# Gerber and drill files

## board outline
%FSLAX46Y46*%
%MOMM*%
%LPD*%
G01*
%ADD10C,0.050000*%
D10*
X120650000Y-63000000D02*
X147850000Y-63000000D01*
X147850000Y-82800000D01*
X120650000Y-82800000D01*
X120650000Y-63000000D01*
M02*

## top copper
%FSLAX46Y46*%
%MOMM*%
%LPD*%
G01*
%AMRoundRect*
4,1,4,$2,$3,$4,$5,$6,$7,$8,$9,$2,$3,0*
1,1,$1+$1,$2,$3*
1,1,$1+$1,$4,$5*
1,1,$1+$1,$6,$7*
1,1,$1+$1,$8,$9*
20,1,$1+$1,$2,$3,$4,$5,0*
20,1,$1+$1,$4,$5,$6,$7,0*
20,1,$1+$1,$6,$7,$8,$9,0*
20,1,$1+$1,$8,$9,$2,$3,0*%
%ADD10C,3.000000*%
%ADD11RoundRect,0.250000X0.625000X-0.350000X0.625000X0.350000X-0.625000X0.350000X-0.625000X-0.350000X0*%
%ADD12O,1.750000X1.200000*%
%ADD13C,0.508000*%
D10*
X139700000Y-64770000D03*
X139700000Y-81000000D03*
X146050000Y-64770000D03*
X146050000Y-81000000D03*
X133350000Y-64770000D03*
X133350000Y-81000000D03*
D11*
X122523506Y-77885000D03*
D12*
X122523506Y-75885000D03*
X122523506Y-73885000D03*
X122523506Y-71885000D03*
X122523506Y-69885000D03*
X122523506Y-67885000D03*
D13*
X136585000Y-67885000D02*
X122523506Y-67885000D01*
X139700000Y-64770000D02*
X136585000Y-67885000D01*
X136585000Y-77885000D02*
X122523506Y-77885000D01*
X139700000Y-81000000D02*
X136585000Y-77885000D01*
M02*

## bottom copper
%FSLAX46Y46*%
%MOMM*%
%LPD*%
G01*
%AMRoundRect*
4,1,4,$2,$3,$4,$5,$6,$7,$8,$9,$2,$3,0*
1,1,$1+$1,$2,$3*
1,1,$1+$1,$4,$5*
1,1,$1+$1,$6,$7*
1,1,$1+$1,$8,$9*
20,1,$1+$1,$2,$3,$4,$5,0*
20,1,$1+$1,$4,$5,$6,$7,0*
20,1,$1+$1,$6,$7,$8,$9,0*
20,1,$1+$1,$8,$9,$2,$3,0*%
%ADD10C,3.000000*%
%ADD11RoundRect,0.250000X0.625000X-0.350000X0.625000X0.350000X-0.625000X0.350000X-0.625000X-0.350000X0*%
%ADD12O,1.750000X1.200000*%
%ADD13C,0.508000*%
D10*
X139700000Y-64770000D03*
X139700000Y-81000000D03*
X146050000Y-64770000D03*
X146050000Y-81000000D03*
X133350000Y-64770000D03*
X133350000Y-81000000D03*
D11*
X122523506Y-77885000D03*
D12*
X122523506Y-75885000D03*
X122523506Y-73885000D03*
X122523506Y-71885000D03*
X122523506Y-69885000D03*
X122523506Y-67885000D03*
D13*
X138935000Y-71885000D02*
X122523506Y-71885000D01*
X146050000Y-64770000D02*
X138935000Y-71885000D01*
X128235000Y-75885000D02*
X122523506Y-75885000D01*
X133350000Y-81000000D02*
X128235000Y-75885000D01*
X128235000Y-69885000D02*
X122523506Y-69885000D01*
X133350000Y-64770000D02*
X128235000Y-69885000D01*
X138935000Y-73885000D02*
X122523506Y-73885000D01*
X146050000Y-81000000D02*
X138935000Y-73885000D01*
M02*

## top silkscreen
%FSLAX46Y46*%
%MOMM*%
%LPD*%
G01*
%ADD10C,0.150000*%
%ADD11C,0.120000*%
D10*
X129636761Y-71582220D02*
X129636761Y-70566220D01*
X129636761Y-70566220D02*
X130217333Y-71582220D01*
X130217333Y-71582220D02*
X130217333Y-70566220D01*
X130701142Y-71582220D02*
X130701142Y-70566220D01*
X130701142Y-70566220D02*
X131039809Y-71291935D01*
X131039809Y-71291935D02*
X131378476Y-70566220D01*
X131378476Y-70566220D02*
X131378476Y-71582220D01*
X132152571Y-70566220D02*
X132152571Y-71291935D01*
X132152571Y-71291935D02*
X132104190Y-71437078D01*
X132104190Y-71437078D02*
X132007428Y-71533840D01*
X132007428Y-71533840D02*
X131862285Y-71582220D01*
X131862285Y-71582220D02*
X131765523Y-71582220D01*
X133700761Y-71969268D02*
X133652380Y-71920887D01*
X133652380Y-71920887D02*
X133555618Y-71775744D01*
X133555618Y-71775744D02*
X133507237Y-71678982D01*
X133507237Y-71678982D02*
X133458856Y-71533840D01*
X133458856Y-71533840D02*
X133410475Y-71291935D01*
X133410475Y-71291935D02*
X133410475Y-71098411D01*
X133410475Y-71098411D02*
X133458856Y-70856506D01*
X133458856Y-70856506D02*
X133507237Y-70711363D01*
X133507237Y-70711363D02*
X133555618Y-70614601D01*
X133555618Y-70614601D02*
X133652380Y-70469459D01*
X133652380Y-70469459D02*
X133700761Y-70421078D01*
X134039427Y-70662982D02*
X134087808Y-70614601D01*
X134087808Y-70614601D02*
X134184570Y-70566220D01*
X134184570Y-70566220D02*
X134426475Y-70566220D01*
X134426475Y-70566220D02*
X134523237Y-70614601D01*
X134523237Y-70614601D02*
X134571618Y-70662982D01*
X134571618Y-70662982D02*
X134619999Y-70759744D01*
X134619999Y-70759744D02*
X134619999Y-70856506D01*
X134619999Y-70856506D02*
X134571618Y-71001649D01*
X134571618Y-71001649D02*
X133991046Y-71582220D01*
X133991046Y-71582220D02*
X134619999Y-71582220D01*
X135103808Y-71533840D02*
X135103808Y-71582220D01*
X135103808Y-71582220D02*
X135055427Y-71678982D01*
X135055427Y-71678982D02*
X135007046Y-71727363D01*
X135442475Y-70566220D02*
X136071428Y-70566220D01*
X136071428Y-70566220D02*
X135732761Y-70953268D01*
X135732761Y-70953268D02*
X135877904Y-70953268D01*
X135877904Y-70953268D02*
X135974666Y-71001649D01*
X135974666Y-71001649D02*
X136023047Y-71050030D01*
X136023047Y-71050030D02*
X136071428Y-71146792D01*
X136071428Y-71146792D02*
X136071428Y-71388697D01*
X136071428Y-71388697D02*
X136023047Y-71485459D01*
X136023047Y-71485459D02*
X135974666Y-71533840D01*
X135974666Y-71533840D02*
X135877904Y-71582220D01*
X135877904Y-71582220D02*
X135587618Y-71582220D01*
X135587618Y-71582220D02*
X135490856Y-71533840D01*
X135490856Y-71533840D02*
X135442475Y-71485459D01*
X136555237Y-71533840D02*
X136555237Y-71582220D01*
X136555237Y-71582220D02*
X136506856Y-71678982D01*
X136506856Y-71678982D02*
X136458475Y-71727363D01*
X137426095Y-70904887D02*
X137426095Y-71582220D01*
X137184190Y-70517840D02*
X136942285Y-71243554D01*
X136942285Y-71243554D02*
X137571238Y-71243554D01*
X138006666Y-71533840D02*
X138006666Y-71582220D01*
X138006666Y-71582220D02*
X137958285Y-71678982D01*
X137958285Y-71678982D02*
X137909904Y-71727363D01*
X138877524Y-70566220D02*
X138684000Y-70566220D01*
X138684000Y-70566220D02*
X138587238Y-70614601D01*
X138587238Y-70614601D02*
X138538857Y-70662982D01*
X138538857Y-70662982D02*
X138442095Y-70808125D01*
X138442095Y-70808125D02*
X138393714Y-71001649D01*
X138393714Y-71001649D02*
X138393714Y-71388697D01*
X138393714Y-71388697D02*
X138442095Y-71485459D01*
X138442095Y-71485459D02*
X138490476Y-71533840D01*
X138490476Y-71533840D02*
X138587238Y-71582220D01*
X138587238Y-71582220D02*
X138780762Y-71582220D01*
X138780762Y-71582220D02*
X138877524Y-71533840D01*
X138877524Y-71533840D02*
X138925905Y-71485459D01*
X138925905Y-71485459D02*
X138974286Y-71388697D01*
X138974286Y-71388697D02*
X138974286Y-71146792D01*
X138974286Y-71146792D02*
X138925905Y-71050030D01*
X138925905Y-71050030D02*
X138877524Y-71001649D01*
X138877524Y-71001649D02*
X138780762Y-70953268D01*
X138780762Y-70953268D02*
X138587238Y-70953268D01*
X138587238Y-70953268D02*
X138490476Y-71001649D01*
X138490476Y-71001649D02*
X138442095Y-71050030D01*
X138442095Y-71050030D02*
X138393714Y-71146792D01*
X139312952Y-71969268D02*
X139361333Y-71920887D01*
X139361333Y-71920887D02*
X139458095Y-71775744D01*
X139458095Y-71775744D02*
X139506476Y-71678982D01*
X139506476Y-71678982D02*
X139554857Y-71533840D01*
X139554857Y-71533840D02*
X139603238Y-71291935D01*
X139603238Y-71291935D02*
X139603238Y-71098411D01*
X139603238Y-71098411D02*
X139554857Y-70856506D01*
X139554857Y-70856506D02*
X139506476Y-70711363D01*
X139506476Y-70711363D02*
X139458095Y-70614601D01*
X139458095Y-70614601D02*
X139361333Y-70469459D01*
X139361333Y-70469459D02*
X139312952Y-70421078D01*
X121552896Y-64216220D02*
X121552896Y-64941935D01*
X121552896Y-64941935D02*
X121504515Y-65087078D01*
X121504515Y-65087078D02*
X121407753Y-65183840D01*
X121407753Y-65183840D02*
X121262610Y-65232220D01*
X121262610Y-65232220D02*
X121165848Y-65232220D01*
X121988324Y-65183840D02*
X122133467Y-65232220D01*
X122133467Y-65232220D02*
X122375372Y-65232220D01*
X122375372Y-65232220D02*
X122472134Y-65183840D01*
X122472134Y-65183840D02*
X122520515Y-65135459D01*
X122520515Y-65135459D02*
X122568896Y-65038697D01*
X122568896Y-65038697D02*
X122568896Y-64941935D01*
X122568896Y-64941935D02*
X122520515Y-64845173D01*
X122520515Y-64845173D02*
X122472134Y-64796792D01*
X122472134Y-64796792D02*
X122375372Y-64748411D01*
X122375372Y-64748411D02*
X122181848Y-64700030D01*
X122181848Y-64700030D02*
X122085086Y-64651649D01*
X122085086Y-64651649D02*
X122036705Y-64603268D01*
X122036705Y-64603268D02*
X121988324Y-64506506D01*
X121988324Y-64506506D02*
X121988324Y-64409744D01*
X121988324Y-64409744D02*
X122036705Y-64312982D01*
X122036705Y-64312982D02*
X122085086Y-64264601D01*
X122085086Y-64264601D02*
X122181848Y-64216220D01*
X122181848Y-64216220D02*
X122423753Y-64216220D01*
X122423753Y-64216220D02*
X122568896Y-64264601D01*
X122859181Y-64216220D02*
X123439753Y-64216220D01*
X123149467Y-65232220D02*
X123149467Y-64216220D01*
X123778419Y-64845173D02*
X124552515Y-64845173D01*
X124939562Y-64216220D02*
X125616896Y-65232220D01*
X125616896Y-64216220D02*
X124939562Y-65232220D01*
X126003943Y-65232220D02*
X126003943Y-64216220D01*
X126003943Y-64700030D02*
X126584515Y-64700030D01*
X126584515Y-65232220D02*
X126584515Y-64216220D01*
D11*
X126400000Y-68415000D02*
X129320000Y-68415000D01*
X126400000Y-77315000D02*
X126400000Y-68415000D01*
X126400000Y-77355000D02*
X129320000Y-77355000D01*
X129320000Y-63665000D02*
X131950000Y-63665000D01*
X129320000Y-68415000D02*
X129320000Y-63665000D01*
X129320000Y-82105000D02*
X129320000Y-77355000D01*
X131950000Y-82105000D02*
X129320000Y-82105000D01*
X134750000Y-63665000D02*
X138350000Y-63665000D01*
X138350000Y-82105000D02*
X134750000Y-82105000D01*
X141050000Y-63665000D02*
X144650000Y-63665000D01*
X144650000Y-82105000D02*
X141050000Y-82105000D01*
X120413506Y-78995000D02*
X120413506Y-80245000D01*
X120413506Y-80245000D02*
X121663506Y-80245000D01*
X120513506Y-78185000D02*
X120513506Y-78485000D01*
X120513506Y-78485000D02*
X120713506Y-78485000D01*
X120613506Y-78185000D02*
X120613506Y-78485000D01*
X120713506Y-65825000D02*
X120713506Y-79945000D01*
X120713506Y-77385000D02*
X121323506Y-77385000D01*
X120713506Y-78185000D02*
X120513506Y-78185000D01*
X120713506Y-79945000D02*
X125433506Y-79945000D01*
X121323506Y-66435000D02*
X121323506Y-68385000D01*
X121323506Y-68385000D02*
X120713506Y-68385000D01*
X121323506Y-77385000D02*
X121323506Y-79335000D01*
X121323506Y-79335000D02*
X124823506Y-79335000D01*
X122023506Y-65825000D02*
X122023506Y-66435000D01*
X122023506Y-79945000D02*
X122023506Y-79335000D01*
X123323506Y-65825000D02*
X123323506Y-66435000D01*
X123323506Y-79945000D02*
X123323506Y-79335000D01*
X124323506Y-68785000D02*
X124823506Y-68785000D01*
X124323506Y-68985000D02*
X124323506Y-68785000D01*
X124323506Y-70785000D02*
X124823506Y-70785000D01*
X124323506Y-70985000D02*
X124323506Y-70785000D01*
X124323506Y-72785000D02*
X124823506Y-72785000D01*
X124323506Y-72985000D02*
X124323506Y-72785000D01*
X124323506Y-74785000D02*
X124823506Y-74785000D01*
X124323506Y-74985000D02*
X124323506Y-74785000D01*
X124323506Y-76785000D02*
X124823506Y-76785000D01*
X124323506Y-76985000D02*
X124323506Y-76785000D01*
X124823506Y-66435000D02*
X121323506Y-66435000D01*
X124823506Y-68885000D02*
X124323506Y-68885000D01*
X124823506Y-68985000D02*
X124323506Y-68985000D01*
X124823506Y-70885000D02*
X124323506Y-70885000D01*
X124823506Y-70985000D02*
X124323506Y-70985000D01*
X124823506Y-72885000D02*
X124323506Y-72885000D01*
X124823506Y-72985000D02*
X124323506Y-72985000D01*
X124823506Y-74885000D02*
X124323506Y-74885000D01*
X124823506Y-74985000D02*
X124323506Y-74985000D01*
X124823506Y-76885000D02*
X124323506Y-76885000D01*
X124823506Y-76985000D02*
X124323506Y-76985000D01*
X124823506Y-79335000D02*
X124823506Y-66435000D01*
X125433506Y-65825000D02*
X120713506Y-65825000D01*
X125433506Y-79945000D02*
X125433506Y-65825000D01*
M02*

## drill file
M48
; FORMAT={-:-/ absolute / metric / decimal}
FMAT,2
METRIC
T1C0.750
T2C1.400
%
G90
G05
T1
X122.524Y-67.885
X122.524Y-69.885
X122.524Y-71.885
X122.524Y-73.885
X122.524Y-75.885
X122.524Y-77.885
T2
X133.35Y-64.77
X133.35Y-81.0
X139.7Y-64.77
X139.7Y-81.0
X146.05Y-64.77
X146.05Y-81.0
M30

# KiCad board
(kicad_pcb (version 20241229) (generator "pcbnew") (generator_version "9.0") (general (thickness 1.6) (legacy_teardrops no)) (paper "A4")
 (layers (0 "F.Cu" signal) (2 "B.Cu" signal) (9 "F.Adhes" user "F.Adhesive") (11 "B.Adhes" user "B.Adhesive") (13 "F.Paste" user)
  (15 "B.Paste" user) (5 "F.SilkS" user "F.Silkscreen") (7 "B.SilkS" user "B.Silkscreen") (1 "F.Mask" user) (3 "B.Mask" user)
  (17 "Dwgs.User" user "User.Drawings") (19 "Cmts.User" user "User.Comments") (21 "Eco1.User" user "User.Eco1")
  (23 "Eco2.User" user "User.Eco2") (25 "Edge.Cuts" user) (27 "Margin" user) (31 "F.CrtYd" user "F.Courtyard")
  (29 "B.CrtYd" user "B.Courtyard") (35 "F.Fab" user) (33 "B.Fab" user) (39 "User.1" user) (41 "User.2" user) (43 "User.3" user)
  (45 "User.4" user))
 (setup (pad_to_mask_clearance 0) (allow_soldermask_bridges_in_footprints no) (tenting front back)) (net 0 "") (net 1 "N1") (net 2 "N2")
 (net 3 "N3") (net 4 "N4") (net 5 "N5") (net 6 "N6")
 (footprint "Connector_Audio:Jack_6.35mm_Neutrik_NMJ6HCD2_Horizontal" (layer "F.Cu") (at 133.35 64.77)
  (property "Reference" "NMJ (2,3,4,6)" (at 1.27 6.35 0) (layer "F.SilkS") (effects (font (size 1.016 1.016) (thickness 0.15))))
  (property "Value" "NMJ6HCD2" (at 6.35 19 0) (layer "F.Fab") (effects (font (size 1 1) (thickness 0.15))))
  (fp_line (start -6.95 3.645) (end -4.03 3.645) (stroke (width 0.12) (type solid)) (layer "F.SilkS"))
  (fp_line (start -6.95 12.545) (end -6.95 3.645) (stroke (width 0.12) (type solid)) (layer "F.SilkS"))
  (fp_line (start -6.95 12.585) (end -4.03 12.585) (stroke (width 0.12) (type solid)) (layer "F.SilkS"))
  (fp_line (start -4.03 -1.105) (end -1.4 -1.105) (stroke (width 0.12) (type solid)) (layer "F.SilkS"))
  (fp_line (start -4.03 3.645) (end -4.03 -1.105) (stroke (width 0.12) (type solid)) (layer "F.SilkS"))
  (fp_line (start -4.03 17.335) (end -4.03 12.585) (stroke (width 0.12) (type solid)) (layer "F.SilkS"))
  (fp_line (start -1.4 17.335) (end -4.03 17.335) (stroke (width 0.12) (type solid)) (layer "F.SilkS"))
  (fp_line (start 1.4 -1.105) (end 5 -1.105) (stroke (width 0.12) (type solid)) (layer "F.SilkS"))
  (fp_line (start 5 17.335) (end 1.4 17.335) (stroke (width 0.12) (type solid)) (layer "F.SilkS"))
  (fp_line (start 7.7 -1.105) (end 11.3 -1.105) (stroke (width 0.12) (type solid)) (layer "F.SilkS"))
  (fp_line (start 11.3 17.335) (end 7.7 17.335) (stroke (width 0.12) (type solid)) (layer "F.SilkS"))
  (pad "R" thru_hole circle (at 6.35 0) (size 3 3) (drill 1.4) (layers "*.Cu" "*.Mask") (remove_unused_layers no) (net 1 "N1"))
  (pad "RN" thru_hole circle (at 6.35 16.23) (size 3 3) (drill 1.4) (layers "*.Cu" "*.Mask") (remove_unused_layers no) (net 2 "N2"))
  (pad "S" thru_hole circle (at 12.7 0) (size 3 3) (drill 1.4) (layers "*.Cu" "*.Mask") (remove_unused_layers no) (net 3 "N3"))
  (pad "SN" thru_hole circle (at 12.7 16.23) (size 3 3) (drill 1.4) (layers "*.Cu" "*.Mask") (remove_unused_layers no) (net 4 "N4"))
  (pad "T" thru_hole circle (at 0 0) (size 3 3) (drill 1.4) (layers "*.Cu" "*.Mask") (remove_unused_layers no) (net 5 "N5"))
  (pad "TN" thru_hole circle (at 0 16.23) (size 3 3) (drill 1.4) (layers "*.Cu" "*.Mask") (remove_unused_layers no) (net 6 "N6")))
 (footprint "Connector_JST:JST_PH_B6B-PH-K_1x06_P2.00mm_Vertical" (layer "F.Cu") (at 122.523506 77.885 90)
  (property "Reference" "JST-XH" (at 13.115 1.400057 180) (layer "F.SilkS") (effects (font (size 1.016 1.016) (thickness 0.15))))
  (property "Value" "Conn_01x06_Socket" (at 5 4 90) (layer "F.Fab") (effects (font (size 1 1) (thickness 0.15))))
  (fp_line (start -1.11 -2.11) (end -2.36 -2.11) (stroke (width 0.12) (type solid)) (layer "F.SilkS"))
  (fp_line (start -2.36 -2.11) (end -2.36 -0.86) (stroke (width 0.12) (type solid)) (layer "F.SilkS"))
  (fp_line (start -0.3 -2.01) (end -0.6 -2.01) (stroke (width 0.12) (type solid)) (layer "F.SilkS"))
  (fp_line (start -0.6 -2.01) (end -0.6 -1.81) (stroke (width 0.12) (type solid)) (layer "F.SilkS"))
  (fp_line (start -0.3 -1.91) (end -0.6 -1.91) (stroke (width 0.12) (type solid)) (layer "F.SilkS"))
  (fp_line (start 12.06 -1.81) (end -2.06 -1.81) (stroke (width 0.12) (type solid)) (layer "F.SilkS"))
  (fp_line (start 0.5 -1.81) (end 0.5 -1.2) (stroke (width 0.12) (type solid)) (layer "F.SilkS"))
  (fp_line (start -0.3 -1.81) (end -0.3 -2.01) (stroke (width 0.12) (type solid)) (layer "F.SilkS"))
  (fp_line (start -2.06 -1.81) (end -2.06 2.91) (stroke (width 0.12) (type solid)) (layer "F.SilkS"))
  (fp_line (start 11.45 -1.2) (end 9.5 -1.2) (stroke (width 0.12) (type solid)) (layer "F.SilkS"))
  (fp_line (start 9.5 -1.2) (end 9.5 -1.81) (stroke (width 0.12) (type solid)) (layer "F.SilkS"))
  (fp_line (start 0.5 -1.2) (end -1.45 -1.2) (stroke (width 0.12) (type solid)) (layer "F.SilkS"))
  (fp_line (start -1.45 -1.2) (end -1.45 2.3) (stroke (width 0.12) (type solid)) (layer "F.SilkS"))
  (fp_line (start 12.06 -0.5) (end 11.45 -0.5) (stroke (width 0.12) (type solid)) (layer "F.SilkS"))
  (fp_line (start -2.06 -0.5) (end -1.45 -0.5) (stroke (width 0.12) (type solid)) (layer "F.SilkS"))
  (fp_line (start 12.06 0.8) (end 11.45 0.8) (stroke (width 0.12) (type solid)) (layer "F.SilkS"))
  (fp_line (start -2.06 0.8) (end -1.45 0.8) (stroke (width 0.12) (type solid)) (layer "F.SilkS"))
  (fp_line (start 9.1 1.8) (end 9.1 2.3) (stroke (width 0.12) (type solid)) (layer "F.SilkS"))
  (fp_line (start 8.9 1.8) (end 9.1 1.8) (stroke (width 0.12) (type solid)) (layer "F.SilkS"))
  (fp_line (start 7.1 1.8) (end 7.1 2.3) (stroke (width 0.12) (type solid)) (layer "F.SilkS"))
  (fp_line (start 6.9 1.8) (end 7.1 1.8) (stroke (width 0.12) (type solid)) (layer "F.SilkS"))
  (fp_line (start 5.1 1.8) (end 5.1 2.3) (stroke (width 0.12) (type solid)) (layer "F.SilkS"))
  (fp_line (start 4.9 1.8) (end 5.1 1.8) (stroke (width 0.12) (type solid)) (layer "F.SilkS"))
  (fp_line (start 3.1 1.8) (end 3.1 2.3) (stroke (width 0.12) (type solid)) (layer "F.SilkS"))
  (fp_line (start 2.9 1.8) (end 3.1 1.8) (stroke (width 0.12) (type solid)) (layer "F.SilkS"))
  (fp_line (start 1.1 1.8) (end 1.1 2.3) (stroke (width 0.12) (type solid)) (layer "F.SilkS"))
  (fp_line (start 0.9 1.8) (end 1.1 1.8) (stroke (width 0.12) (type solid)) (layer "F.SilkS"))
  (fp_line (start 11.45 2.3) (end 11.45 -1.2) (stroke (width 0.12) (type solid)) (layer "F.SilkS"))
  (fp_line (start 9 2.3) (end 9 1.8) (stroke (width 0.12) (type solid)) (layer "F.SilkS"))
  (fp_line (start 8.9 2.3) (end 8.9 1.8) (stroke (width 0.12) (type solid)) (layer "F.SilkS"))
  (fp_line (start 7 2.3) (end 7 1.8) (stroke (width 0.12) (type solid)) (layer "F.SilkS"))
  (fp_line (start 6.9 2.3) (end 6.9 1.8) (stroke (width 0.12) (type solid)) (layer "F.SilkS"))
  (fp_line (start 5 2.3) (end 5 1.8) (stroke (width 0.12) (type solid)) (layer "F.SilkS"))
  (fp_line (start 4.9 2.3) (end 4.9 1.8) (stroke (width 0.12) (type solid)) (layer "F.SilkS"))
  (fp_line (start 3 2.3) (end 3 1.8) (stroke (width 0.12) (type solid)) (layer "F.SilkS"))
  (fp_line (start 2.9 2.3) (end 2.9 1.8) (stroke (width 0.12) (type solid)) (layer "F.SilkS"))
  (fp_line (start 1 2.3) (end 1 1.8) (stroke (width 0.12) (type solid)) (layer "F.SilkS"))
  (fp_line (start 0.9 2.3) (end 0.9 1.8) (stroke (width 0.12) (type solid)) (layer "F.SilkS"))
  (fp_line (start -1.45 2.3) (end 11.45 2.3) (stroke (width 0.12) (type solid)) (layer "F.SilkS"))
  (fp_line (start 12.06 2.91) (end 12.06 -1.81) (stroke (width 0.12) (type solid)) (layer "F.SilkS"))
  (fp_line (start -2.06 2.91) (end 12.06 2.91) (stroke (width 0.12) (type solid)) (layer "F.SilkS"))
  (pad "1" thru_hole roundrect (at 0 0 90) (size 1.2 1.75) (drill 0.75) (layers "*.Cu" "*.Mask") (remove_unused_layers no)
   (roundrect_rratio 0.208333) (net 2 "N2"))
  (pad "2" thru_hole oval (at 2 0 90) (size 1.2 1.75) (drill 0.75) (layers "*.Cu" "*.Mask") (remove_unused_layers no) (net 6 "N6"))
  (pad "3" thru_hole oval (at 4 0 90) (size 1.2 1.75) (drill 0.75) (layers "*.Cu" "*.Mask") (remove_unused_layers no) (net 4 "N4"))
  (pad "4" thru_hole oval (at 6 0 90) (size 1.2 1.75) (drill 0.75) (layers "*.Cu" "*.Mask") (remove_unused_layers no) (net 3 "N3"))
  (pad "5" thru_hole oval (at 8 0 90) (size 1.2 1.75) (drill 0.75) (layers "*.Cu" "*.Mask") (remove_unused_layers no) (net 5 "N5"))
  (pad "6" thru_hole oval (at 10 0 90) (size 1.2 1.75) (drill 0.75) (layers "*.Cu" "*.Mask") (remove_unused_layers no) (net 1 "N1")))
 (gr_rect (start 120.65 63) (end 147.85 82.8) (stroke (width 0.05) (type solid)) (fill no) (layer "Edge.Cuts"))
 (segment (start 138.935 71.885) (end 122.523506 71.885) (width 0.508) (layer "B.Cu") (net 3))
 (segment (start 146.05 64.77) (end 138.935 71.885) (width 0.508) (layer "B.Cu") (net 3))
 (segment (start 136.585 67.885) (end 122.523506 67.885) (width 0.508) (layer "F.Cu") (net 1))
 (segment (start 139.7 64.77) (end 136.585 67.885) (width 0.508) (layer "F.Cu") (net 1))
 (segment (start 128.235 75.885) (end 122.523506 75.885) (width 0.508) (layer "B.Cu") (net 6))
 (segment (start 133.35 81) (end 128.235 75.885) (width 0.508) (layer "B.Cu") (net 6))
 (segment (start 136.585 77.885) (end 122.523506 77.885) (width 0.508) (layer "F.Cu") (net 2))
 (segment (start 139.7 81) (end 136.585 77.885) (width 0.508) (layer "F.Cu") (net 2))
 (segment (start 128.235 69.885) (end 122.523506 69.885) (width 0.508) (layer "B.Cu") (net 5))
 (segment (start 133.35 64.77) (end 128.235 69.885) (width 0.508) (layer "B.Cu") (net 5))
 (segment (start 138.935 73.885) (end 122.523506 73.885) (width 0.508) (layer "B.Cu") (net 4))
 (segment (start 146.05 81) (end 138.935 73.885) (width 0.508) (layer "B.Cu") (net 4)))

